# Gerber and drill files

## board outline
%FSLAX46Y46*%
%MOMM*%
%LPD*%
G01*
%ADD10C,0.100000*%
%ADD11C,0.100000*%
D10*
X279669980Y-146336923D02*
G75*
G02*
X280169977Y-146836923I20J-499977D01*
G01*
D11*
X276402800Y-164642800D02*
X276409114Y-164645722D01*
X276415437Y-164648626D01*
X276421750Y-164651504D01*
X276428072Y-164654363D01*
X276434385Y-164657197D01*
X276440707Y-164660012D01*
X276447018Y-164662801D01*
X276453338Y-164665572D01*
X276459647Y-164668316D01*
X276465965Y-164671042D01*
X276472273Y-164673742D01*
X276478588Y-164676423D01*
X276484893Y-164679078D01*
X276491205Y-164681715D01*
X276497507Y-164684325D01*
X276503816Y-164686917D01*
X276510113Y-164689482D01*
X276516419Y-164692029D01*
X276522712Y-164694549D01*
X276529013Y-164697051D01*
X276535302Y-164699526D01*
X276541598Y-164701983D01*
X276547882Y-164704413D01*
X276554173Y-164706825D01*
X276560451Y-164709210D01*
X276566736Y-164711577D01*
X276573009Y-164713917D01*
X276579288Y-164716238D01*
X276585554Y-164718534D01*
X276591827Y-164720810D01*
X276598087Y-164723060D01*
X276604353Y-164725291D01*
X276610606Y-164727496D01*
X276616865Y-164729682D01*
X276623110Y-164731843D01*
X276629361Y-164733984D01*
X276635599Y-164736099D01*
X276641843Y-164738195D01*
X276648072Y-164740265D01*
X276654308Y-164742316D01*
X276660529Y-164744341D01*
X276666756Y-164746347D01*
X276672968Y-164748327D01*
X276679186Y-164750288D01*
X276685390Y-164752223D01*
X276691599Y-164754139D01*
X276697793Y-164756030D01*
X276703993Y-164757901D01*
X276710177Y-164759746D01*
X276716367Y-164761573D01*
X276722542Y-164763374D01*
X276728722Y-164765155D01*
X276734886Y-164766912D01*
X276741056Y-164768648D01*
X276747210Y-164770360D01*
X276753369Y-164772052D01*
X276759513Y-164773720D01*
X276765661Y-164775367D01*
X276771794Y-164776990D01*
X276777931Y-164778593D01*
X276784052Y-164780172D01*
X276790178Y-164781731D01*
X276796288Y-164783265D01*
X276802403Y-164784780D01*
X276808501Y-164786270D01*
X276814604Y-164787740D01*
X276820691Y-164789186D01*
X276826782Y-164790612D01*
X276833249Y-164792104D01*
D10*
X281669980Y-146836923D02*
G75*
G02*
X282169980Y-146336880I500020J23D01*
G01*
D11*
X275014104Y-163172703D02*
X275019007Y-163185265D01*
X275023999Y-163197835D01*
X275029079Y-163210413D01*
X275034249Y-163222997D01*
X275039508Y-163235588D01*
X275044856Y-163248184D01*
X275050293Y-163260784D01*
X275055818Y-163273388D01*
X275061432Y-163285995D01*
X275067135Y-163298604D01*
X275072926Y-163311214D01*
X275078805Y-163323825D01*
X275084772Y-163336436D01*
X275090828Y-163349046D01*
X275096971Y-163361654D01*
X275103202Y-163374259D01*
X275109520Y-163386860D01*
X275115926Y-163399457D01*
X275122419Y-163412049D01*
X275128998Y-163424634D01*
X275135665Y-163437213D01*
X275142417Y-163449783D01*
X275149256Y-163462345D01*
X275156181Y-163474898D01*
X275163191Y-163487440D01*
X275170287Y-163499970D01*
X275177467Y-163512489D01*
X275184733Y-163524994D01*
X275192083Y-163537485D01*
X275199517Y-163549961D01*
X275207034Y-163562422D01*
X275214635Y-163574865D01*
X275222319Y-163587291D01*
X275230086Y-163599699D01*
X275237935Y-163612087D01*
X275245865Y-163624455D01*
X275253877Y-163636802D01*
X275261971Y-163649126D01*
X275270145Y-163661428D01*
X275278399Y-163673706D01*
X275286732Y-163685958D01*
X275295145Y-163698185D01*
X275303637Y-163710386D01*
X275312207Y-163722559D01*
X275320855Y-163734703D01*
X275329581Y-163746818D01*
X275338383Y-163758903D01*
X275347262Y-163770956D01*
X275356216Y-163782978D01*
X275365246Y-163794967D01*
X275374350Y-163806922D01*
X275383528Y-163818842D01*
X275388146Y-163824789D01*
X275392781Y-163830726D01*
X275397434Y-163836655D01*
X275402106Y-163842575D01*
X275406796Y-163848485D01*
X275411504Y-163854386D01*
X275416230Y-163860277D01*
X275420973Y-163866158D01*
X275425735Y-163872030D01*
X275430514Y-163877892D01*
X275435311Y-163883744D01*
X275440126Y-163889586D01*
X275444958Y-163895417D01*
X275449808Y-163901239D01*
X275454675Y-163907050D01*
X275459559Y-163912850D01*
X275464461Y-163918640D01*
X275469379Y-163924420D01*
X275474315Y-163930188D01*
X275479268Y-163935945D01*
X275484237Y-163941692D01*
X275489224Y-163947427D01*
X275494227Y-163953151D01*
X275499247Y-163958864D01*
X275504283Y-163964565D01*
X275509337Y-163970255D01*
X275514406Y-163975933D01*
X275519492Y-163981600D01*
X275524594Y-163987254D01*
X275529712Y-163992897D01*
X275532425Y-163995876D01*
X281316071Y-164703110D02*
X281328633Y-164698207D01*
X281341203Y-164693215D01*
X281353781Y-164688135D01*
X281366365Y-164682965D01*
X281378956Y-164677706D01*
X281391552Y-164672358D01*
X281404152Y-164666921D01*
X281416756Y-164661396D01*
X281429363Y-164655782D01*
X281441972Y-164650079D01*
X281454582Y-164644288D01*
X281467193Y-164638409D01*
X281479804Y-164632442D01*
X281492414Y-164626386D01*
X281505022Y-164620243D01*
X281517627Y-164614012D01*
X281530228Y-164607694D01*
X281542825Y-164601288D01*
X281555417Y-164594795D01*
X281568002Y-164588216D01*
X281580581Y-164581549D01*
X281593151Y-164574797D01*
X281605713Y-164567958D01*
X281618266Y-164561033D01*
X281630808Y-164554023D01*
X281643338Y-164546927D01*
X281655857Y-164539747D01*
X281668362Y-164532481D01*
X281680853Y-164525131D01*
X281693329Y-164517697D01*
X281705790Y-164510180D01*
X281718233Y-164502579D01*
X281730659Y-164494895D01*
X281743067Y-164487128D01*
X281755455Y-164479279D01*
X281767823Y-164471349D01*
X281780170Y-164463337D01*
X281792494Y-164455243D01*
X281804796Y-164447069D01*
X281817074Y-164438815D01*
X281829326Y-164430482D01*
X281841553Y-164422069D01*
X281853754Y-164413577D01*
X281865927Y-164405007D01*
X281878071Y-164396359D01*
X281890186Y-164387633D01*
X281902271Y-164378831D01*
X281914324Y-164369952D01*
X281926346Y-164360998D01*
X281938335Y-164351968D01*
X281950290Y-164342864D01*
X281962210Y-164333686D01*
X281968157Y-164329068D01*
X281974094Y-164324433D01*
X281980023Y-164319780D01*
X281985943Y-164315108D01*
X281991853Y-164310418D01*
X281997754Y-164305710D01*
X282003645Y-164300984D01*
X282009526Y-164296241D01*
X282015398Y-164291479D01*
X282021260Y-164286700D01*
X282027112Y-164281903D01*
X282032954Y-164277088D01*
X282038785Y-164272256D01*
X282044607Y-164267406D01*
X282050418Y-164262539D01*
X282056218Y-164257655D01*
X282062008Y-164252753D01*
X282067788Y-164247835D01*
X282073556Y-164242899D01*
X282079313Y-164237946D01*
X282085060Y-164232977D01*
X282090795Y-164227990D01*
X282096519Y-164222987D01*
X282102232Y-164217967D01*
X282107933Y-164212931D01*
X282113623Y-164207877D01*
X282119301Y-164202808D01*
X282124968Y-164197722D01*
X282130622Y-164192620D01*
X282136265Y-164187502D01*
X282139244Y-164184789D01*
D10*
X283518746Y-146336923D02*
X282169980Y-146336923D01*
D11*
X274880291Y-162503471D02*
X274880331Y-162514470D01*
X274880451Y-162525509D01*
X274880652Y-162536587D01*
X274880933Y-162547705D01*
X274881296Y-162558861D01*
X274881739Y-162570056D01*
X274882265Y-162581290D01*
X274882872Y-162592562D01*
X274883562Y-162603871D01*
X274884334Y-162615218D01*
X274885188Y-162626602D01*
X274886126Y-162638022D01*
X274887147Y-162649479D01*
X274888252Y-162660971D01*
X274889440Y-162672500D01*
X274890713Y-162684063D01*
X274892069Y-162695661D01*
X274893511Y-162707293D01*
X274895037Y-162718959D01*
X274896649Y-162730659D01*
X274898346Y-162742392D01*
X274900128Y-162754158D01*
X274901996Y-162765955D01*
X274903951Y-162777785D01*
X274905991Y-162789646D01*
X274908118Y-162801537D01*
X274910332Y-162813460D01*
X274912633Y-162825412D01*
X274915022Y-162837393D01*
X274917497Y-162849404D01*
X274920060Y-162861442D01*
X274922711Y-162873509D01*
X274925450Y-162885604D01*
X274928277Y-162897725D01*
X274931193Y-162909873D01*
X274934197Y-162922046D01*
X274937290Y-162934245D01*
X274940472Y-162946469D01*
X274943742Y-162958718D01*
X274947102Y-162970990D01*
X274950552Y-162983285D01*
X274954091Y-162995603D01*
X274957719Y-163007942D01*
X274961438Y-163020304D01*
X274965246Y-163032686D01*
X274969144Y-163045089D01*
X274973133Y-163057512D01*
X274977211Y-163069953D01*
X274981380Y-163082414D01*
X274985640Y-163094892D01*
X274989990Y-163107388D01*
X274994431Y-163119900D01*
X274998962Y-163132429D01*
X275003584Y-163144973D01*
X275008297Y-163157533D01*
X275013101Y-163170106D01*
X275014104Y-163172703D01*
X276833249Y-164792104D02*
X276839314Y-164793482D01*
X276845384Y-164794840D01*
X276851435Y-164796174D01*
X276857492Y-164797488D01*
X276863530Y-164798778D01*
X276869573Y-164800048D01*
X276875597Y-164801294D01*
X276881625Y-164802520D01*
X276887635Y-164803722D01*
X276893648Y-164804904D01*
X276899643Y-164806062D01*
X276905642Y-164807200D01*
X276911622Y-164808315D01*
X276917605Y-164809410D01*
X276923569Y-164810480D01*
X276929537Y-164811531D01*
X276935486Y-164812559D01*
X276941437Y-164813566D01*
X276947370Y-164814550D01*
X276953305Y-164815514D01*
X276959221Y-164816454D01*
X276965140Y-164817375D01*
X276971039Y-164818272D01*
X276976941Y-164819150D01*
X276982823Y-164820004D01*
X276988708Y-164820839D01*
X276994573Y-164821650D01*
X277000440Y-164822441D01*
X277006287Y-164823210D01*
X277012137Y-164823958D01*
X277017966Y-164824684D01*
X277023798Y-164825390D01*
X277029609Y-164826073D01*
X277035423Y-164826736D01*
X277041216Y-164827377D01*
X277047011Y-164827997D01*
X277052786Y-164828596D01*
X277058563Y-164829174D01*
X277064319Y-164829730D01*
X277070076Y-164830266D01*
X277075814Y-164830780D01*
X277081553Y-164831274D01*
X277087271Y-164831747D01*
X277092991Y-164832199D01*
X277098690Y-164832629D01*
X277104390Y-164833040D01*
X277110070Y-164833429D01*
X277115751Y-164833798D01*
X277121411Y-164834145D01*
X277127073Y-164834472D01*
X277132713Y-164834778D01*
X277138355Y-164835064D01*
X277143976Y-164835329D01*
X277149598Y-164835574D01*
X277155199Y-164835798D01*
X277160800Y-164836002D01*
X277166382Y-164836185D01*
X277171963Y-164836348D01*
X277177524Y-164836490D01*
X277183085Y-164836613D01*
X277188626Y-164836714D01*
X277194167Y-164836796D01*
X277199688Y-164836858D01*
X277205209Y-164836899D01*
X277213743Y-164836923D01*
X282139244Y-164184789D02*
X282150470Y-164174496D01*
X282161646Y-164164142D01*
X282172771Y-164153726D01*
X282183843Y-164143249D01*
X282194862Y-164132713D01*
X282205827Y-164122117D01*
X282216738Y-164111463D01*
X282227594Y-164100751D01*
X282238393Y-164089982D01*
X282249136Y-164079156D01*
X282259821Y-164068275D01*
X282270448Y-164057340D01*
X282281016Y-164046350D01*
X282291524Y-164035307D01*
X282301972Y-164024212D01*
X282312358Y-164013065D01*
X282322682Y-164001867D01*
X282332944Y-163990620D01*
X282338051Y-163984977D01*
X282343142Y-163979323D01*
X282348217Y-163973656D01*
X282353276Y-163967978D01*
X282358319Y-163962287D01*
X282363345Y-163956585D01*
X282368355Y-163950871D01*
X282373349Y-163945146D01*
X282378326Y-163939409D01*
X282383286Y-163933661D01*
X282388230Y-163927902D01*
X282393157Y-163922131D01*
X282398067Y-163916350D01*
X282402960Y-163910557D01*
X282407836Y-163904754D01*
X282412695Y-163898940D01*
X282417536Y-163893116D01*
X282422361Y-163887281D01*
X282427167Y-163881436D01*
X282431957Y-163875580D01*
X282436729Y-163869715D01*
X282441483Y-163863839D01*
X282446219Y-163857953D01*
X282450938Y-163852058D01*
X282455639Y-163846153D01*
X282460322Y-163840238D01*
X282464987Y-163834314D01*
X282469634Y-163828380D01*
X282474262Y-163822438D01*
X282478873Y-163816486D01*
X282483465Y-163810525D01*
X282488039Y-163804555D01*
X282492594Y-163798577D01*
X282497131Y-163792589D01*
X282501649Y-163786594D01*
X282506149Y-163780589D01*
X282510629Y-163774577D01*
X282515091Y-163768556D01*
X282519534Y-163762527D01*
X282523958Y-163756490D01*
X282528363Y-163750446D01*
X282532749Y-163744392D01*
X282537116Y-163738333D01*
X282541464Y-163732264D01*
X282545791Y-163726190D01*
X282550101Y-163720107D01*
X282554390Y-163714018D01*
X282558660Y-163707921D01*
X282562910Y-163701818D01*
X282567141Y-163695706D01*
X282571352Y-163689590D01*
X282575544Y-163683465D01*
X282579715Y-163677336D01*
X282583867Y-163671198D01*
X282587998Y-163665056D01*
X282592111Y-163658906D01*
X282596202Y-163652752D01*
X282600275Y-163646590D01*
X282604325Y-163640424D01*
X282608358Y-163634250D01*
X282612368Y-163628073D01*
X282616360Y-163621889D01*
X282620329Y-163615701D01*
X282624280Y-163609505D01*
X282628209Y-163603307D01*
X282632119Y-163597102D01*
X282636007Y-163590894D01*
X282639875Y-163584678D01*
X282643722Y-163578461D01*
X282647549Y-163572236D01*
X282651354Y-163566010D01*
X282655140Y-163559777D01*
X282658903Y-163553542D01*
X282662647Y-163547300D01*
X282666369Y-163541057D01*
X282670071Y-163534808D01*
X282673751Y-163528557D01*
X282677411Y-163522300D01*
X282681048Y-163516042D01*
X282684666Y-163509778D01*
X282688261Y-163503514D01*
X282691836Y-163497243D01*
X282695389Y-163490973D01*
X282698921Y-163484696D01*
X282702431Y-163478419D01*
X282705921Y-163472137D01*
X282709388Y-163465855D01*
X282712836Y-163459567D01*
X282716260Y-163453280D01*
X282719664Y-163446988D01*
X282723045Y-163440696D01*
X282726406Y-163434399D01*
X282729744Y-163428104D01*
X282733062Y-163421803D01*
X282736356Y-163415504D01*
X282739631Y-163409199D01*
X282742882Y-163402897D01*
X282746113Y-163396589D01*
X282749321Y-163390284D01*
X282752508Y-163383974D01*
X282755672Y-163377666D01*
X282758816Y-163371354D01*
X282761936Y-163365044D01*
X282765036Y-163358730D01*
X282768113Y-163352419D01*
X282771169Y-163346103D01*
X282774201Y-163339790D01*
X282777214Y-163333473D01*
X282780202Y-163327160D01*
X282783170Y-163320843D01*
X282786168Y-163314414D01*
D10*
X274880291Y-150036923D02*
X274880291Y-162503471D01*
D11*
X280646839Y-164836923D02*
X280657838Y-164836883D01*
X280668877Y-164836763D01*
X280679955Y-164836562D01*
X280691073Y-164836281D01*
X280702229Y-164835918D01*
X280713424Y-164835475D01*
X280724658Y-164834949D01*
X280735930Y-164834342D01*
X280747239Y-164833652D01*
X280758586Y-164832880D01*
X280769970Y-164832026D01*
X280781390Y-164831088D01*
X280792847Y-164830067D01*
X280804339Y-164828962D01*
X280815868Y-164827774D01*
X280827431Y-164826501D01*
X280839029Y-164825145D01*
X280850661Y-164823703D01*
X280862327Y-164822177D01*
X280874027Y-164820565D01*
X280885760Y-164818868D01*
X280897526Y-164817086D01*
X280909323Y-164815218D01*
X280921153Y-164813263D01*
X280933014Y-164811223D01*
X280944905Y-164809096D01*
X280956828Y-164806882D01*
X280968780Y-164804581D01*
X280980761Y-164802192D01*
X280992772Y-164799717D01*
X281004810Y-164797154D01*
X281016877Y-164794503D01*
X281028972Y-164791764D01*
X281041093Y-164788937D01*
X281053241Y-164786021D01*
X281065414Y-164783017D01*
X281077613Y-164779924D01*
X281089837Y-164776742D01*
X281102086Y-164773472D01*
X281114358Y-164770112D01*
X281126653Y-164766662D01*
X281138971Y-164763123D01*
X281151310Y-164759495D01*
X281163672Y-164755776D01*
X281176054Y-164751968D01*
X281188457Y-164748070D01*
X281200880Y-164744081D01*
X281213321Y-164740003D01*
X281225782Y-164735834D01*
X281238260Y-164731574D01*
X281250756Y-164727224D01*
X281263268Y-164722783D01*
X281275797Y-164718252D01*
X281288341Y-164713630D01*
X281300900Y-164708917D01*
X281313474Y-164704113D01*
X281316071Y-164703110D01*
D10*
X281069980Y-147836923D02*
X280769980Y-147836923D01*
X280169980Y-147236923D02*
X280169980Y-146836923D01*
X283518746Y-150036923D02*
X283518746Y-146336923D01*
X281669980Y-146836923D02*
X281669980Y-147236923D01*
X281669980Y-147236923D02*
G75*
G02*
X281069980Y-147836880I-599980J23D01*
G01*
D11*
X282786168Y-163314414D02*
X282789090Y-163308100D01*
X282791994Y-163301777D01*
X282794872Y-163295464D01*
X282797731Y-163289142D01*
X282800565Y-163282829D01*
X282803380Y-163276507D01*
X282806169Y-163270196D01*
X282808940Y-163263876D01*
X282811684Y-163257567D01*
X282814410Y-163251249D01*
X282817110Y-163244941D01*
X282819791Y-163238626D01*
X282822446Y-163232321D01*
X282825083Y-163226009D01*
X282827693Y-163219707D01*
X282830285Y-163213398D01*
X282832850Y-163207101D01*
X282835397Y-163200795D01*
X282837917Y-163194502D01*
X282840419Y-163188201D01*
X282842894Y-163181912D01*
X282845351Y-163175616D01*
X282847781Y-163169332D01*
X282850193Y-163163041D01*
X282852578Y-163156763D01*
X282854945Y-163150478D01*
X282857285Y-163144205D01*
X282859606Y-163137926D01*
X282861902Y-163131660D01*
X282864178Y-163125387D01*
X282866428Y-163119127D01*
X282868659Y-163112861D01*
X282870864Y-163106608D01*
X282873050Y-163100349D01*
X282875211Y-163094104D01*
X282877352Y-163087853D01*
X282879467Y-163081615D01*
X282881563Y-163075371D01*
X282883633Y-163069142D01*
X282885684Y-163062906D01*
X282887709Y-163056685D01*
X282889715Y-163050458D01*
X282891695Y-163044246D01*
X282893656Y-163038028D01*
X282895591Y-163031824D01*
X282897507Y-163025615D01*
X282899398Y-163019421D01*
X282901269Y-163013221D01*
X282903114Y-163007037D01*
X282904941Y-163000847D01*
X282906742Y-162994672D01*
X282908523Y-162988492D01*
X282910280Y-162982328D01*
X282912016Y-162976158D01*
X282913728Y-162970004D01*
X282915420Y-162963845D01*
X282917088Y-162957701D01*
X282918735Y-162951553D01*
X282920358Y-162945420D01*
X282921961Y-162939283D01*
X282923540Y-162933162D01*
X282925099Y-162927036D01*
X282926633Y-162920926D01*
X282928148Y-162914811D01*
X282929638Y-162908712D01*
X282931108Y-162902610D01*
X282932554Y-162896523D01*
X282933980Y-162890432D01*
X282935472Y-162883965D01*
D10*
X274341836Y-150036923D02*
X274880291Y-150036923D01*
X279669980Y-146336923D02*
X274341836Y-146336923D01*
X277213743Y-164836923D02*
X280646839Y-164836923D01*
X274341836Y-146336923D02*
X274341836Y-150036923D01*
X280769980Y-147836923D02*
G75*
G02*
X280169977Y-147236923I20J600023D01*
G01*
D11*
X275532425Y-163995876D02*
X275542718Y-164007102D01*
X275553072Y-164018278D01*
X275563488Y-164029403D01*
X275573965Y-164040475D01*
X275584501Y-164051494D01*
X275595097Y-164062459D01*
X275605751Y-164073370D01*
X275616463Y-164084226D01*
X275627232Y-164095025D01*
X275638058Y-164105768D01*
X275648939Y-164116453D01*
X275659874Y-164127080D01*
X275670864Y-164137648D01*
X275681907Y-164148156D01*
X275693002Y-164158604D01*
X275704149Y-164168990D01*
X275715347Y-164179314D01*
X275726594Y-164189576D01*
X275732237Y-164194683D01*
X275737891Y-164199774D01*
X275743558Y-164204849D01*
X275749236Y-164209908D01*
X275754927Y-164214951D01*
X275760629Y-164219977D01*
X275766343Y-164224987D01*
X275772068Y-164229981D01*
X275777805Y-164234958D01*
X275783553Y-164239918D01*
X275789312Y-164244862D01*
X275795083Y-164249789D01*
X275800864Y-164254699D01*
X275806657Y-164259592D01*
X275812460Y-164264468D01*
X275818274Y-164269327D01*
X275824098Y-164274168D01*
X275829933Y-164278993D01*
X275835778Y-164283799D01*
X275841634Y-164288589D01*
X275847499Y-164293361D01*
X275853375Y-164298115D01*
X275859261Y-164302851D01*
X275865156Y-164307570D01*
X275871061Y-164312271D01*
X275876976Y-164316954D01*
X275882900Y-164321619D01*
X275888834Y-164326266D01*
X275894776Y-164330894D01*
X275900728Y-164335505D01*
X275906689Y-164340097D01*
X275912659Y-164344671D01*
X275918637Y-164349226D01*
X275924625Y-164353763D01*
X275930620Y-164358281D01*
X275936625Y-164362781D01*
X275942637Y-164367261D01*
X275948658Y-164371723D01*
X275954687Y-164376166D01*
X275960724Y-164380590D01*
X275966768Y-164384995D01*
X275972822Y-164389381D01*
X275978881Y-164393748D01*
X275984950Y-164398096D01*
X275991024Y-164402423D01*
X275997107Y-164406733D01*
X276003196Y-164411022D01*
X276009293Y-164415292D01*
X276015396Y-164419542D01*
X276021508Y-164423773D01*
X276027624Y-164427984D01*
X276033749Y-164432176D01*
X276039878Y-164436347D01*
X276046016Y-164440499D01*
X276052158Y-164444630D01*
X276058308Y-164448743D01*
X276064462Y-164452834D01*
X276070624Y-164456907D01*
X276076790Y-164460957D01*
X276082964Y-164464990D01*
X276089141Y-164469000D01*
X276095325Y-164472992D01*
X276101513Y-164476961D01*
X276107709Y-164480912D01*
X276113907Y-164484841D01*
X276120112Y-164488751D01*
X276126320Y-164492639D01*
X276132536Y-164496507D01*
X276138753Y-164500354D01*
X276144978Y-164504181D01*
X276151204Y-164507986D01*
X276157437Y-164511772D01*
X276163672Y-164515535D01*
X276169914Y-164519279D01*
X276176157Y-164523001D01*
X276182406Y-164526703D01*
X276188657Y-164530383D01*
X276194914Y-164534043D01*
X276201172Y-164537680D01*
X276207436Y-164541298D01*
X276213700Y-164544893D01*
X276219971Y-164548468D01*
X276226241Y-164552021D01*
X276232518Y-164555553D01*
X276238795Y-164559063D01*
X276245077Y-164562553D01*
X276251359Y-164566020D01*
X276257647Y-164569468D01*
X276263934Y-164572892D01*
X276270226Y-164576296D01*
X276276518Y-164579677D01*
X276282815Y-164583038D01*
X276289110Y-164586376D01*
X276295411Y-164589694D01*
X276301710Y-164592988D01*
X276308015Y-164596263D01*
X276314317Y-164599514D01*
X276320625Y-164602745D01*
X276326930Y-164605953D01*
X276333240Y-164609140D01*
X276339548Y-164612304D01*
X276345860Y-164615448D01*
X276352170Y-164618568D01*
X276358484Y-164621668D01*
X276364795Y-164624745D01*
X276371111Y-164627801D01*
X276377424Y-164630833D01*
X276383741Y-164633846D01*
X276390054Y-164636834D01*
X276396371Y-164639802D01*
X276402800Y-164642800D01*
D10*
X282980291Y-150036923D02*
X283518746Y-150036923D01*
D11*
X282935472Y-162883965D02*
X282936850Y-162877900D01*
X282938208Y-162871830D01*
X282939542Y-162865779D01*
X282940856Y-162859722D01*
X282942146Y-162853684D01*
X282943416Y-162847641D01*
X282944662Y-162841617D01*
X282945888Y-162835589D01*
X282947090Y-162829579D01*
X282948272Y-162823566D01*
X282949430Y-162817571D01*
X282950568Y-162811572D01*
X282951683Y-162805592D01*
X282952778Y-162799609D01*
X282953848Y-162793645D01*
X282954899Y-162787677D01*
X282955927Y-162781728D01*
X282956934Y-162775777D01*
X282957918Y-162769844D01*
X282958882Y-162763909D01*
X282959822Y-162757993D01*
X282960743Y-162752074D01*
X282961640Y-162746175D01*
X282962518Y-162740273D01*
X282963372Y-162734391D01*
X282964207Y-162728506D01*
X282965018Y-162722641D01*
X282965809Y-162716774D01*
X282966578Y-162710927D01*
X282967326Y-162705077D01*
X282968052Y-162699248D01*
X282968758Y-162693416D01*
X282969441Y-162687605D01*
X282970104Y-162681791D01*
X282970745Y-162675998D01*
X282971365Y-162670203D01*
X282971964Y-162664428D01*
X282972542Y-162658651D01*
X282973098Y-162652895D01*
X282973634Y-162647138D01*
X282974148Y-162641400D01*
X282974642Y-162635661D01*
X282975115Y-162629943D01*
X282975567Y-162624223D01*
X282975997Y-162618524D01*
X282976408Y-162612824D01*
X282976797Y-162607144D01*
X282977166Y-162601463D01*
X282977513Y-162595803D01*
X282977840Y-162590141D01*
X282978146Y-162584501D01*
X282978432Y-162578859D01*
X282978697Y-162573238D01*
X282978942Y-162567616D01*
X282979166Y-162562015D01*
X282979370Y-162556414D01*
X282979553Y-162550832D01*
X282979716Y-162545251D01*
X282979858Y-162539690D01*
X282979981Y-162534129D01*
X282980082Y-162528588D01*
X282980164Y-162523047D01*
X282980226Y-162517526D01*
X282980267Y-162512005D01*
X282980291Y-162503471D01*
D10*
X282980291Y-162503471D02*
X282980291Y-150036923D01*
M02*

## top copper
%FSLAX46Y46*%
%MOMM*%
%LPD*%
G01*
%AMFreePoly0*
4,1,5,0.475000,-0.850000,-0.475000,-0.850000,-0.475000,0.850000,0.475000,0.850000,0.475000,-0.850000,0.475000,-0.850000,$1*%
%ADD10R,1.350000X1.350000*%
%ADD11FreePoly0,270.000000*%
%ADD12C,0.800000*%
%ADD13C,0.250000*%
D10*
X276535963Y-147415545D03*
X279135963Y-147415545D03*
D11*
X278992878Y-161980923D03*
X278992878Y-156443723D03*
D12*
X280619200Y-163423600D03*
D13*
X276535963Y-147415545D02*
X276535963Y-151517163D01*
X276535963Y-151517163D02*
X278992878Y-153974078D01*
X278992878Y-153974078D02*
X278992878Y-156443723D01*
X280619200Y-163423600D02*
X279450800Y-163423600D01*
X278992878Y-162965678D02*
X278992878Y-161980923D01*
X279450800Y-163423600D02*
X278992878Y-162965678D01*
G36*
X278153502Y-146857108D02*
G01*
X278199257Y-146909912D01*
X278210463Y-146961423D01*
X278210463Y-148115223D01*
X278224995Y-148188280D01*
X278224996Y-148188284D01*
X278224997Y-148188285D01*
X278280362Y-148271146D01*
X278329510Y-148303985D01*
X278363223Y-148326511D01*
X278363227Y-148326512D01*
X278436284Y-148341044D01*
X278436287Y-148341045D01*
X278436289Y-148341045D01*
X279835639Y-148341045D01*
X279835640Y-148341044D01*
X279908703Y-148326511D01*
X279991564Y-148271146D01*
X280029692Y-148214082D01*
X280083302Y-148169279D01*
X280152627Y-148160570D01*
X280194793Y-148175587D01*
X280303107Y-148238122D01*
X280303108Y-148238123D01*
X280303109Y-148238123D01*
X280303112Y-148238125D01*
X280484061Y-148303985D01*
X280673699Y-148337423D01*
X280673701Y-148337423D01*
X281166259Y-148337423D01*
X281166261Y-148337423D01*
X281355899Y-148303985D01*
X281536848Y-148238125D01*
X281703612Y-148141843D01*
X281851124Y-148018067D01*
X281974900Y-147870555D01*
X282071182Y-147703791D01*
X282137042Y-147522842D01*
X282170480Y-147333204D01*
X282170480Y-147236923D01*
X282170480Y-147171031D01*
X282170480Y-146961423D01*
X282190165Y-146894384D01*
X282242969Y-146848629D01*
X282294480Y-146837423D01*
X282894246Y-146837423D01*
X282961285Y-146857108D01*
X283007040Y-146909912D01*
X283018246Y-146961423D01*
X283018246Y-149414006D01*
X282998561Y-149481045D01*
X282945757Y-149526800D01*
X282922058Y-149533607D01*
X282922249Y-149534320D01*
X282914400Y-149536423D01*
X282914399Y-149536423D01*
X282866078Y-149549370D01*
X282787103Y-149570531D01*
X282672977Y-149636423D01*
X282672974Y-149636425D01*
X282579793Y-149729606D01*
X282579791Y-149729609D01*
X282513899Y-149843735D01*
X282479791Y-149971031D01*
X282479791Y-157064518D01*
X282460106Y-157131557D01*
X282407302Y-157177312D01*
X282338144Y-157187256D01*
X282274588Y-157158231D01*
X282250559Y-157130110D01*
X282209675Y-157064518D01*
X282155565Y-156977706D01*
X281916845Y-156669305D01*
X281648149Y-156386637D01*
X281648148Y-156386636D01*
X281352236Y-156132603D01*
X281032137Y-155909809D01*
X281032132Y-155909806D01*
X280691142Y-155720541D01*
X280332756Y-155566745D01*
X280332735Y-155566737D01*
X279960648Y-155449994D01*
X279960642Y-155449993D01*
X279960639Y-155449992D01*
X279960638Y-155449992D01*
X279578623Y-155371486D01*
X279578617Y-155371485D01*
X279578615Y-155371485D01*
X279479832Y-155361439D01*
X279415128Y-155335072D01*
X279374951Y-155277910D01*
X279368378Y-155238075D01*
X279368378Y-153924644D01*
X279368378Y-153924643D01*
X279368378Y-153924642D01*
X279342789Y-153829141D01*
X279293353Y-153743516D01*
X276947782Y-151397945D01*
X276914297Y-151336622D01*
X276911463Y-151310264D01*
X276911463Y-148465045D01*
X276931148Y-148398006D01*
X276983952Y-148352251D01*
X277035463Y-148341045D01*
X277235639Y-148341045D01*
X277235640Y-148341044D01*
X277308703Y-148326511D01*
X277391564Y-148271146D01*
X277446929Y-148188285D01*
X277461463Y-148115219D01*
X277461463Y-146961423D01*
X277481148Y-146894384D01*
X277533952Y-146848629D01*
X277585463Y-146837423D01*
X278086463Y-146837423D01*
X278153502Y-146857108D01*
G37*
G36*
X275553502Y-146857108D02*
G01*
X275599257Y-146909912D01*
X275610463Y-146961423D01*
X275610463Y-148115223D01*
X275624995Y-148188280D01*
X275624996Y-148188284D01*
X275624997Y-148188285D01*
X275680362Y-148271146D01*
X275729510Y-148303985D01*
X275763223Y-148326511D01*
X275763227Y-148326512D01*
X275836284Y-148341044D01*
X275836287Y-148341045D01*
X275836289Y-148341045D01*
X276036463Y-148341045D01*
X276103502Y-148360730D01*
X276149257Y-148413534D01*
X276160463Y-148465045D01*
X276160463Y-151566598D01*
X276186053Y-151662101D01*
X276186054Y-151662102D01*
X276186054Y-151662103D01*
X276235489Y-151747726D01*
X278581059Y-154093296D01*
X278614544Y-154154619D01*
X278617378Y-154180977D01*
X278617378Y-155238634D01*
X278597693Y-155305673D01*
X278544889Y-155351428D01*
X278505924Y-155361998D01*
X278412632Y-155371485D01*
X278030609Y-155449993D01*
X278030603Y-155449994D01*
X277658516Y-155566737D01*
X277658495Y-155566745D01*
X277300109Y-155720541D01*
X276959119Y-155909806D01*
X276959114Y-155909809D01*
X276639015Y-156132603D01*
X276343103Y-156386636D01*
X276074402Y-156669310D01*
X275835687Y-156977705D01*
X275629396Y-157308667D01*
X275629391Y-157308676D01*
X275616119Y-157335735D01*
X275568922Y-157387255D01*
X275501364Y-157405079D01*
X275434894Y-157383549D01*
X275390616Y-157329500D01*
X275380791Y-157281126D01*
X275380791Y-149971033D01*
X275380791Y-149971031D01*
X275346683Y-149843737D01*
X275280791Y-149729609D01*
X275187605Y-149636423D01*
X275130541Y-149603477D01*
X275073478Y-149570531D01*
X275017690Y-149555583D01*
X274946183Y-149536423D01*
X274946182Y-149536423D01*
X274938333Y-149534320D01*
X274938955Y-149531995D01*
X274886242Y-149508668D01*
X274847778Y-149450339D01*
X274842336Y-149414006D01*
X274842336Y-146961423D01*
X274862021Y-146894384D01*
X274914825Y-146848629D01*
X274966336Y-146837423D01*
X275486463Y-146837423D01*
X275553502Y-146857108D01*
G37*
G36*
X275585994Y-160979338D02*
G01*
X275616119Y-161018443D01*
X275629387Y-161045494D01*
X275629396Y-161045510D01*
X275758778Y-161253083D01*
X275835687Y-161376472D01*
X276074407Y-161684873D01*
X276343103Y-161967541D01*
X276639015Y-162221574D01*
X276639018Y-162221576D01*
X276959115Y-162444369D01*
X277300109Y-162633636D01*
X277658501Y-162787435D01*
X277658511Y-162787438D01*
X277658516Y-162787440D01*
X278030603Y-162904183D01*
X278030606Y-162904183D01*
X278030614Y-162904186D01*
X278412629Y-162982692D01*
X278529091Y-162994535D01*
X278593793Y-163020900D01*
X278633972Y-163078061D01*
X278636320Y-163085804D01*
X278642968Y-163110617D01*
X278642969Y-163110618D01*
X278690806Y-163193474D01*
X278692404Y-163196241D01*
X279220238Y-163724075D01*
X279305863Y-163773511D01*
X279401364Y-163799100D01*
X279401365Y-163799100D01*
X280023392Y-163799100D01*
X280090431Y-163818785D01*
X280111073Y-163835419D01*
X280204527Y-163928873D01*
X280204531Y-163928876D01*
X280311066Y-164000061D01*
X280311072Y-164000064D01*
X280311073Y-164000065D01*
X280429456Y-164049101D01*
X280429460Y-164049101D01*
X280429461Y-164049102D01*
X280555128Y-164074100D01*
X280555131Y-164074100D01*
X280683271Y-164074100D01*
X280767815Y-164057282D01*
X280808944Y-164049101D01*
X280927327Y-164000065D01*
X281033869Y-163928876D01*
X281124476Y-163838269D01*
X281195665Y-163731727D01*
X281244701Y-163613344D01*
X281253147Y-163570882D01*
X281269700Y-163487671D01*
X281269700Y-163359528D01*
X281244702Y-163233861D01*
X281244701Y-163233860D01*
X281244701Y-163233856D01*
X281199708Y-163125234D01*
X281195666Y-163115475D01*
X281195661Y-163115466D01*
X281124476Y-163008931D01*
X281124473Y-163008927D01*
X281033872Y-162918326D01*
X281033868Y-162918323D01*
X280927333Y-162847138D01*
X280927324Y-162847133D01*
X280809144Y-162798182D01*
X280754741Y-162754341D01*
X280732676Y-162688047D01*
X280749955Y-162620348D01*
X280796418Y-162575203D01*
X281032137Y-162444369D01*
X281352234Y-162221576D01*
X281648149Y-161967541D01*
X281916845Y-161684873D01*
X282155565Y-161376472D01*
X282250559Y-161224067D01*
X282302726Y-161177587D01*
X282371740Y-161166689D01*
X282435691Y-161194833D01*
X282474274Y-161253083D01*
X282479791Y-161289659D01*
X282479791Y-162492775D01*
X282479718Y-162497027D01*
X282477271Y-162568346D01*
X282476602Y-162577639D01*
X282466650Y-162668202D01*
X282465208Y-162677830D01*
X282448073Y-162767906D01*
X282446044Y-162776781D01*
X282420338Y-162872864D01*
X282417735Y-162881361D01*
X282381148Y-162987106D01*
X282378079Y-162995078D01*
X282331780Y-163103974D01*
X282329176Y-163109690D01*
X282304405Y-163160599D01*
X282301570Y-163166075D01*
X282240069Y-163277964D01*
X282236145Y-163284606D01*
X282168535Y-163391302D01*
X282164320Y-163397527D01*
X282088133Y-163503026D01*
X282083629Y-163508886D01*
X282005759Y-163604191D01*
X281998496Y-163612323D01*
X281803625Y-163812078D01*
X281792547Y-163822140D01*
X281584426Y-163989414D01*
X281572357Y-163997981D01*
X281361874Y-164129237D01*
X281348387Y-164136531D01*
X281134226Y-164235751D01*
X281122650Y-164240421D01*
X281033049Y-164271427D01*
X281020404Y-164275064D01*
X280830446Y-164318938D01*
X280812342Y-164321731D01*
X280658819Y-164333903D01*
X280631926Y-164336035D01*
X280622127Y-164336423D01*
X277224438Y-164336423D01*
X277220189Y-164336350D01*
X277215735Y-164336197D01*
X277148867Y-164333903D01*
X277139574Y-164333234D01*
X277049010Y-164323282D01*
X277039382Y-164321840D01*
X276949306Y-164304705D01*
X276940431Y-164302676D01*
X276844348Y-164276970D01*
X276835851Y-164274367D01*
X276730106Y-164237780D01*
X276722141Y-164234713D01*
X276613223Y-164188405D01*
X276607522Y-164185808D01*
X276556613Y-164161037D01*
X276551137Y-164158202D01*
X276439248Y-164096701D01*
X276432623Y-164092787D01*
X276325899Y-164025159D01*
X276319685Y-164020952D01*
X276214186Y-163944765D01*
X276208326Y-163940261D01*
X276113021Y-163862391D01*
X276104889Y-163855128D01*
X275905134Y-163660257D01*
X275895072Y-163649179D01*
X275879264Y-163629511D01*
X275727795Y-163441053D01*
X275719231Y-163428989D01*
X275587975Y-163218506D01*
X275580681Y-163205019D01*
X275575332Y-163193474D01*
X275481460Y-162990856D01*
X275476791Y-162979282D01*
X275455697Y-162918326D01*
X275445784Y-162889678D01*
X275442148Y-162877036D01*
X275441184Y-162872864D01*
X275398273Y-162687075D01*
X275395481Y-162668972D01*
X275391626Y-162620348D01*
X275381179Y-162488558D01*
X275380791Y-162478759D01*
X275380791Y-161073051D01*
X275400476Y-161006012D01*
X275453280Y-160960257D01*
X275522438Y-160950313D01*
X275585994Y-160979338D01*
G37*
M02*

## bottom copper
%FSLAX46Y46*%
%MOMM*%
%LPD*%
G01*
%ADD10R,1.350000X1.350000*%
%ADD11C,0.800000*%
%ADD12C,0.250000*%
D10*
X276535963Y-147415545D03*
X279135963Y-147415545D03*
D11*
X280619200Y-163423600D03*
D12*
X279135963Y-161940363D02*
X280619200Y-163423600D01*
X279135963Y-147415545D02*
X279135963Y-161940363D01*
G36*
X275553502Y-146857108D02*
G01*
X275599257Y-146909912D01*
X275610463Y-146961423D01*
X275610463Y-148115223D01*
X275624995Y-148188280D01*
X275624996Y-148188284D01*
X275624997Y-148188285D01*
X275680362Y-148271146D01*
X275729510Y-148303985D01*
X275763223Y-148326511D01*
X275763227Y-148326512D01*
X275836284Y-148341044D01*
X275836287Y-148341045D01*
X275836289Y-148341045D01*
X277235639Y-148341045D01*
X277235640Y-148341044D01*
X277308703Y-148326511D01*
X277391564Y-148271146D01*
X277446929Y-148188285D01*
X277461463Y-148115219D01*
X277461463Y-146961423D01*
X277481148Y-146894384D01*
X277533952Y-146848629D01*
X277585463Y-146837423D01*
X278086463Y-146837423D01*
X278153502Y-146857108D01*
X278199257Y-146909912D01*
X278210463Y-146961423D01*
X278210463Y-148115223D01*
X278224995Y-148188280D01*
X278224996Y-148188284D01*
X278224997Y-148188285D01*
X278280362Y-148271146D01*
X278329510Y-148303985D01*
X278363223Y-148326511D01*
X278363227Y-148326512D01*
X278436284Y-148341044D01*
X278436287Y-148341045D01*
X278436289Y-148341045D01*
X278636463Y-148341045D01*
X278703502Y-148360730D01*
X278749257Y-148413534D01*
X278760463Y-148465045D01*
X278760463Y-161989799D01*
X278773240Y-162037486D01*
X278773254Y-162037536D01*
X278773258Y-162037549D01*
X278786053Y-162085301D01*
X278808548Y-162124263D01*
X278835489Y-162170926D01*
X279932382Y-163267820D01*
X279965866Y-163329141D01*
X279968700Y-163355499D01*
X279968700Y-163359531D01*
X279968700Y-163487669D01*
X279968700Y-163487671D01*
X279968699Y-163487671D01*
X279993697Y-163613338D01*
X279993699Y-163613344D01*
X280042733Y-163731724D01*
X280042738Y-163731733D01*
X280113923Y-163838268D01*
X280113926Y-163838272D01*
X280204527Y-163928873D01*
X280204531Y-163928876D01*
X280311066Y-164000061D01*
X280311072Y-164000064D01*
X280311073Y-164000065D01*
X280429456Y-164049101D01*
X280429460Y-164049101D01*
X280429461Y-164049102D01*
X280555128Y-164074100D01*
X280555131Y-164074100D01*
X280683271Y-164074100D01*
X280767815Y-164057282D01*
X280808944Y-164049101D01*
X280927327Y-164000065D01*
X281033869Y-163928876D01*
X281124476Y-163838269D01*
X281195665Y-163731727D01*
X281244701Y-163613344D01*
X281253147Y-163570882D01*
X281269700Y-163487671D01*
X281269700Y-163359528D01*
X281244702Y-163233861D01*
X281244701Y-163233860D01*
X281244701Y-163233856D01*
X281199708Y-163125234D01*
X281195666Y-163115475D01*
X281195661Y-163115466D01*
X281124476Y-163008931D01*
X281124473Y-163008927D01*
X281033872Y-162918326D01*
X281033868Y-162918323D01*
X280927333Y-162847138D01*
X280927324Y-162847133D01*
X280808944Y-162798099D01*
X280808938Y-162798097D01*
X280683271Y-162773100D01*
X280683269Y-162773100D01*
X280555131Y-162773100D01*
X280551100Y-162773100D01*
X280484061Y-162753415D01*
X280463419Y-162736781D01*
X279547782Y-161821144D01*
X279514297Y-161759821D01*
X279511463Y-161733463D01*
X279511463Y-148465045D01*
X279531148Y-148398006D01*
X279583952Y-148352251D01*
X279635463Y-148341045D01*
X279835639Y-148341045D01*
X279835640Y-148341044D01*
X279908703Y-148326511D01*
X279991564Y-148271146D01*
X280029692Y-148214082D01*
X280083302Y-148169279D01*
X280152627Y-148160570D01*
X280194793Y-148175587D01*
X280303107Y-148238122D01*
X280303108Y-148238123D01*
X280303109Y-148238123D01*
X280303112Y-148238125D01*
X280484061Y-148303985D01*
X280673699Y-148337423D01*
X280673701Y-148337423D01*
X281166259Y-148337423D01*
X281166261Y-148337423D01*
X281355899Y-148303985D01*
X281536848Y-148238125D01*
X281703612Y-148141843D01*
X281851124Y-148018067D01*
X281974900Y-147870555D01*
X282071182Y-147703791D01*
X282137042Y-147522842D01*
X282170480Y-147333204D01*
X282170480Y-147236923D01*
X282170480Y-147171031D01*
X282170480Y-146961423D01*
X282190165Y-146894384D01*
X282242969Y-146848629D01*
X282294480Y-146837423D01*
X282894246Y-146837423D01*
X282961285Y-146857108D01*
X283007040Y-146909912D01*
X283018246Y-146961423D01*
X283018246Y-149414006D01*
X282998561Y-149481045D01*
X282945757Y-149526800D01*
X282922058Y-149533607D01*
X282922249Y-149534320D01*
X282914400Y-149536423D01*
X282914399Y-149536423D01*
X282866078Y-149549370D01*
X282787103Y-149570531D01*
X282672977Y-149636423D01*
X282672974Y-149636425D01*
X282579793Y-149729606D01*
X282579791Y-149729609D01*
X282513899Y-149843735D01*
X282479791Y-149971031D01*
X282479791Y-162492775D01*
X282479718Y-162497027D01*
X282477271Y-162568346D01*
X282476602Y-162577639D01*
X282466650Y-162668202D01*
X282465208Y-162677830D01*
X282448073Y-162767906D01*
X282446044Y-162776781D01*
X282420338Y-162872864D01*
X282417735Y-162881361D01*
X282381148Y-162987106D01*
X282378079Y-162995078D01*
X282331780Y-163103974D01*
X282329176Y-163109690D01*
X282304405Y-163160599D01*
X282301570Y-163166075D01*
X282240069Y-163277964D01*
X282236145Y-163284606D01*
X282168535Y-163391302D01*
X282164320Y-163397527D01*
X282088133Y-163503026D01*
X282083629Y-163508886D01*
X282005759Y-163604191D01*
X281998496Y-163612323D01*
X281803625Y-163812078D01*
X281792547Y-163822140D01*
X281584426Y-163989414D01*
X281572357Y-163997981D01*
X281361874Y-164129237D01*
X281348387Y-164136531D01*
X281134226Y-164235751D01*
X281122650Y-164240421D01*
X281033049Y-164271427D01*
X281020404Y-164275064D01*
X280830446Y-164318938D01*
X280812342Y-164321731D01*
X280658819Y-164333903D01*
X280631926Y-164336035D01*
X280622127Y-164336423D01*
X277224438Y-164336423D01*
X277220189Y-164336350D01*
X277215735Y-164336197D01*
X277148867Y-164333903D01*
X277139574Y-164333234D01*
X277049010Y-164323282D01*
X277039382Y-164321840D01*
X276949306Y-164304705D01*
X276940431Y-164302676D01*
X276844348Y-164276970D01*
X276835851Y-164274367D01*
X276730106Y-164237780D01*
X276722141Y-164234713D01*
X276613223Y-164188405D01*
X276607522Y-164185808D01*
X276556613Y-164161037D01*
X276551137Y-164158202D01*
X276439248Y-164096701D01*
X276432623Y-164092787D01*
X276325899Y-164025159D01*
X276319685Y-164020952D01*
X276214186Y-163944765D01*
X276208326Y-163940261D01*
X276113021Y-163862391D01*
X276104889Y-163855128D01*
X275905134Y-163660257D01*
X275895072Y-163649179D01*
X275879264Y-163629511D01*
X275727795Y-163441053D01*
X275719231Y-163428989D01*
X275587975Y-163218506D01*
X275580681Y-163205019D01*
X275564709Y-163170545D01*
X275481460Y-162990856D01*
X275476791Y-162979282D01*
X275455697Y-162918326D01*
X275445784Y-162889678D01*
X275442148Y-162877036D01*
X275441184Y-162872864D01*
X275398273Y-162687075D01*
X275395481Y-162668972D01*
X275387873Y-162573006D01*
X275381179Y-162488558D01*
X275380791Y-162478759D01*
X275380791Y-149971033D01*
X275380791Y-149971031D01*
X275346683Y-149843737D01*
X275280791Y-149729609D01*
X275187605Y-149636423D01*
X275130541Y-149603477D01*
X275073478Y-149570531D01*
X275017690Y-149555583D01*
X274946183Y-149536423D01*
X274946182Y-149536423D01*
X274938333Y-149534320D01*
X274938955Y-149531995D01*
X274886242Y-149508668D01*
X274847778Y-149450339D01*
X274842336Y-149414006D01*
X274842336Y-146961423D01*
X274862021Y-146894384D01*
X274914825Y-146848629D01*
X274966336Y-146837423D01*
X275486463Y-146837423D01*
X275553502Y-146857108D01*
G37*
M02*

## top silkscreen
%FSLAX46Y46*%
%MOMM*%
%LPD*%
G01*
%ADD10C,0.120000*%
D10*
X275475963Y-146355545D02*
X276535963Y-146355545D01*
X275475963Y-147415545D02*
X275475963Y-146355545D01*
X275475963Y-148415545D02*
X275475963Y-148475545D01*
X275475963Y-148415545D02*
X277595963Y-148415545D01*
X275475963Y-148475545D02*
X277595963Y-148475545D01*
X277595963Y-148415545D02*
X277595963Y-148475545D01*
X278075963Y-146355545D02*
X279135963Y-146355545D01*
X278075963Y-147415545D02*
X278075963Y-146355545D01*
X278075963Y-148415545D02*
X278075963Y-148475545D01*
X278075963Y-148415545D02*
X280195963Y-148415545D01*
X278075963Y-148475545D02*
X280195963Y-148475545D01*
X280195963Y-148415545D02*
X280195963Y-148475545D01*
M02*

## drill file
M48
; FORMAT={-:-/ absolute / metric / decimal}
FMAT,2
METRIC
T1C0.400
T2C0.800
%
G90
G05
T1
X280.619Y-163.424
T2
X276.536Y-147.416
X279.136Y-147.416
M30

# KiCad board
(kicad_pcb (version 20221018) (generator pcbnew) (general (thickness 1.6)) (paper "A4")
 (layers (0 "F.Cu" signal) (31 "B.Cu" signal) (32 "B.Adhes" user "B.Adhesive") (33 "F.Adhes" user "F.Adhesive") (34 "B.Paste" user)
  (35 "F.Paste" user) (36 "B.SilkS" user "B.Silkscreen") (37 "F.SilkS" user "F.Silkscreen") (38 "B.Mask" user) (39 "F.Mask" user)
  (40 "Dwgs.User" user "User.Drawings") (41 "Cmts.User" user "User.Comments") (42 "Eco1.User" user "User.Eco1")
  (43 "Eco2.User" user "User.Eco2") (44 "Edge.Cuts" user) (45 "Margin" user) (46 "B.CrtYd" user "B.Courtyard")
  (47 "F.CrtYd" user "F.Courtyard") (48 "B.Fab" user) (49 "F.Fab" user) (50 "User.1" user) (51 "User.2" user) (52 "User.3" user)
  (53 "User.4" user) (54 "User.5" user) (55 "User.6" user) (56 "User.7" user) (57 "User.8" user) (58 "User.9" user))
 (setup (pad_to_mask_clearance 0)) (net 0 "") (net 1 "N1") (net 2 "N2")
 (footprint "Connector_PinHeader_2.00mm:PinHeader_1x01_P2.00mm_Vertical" (layer "F.Cu") (at 276.535963 147.415545)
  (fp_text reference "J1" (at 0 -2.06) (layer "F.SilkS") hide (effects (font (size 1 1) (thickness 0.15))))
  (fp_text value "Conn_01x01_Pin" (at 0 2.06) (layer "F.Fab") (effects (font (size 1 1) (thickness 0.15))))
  (fp_line (start -1.06 -1.06) (end 0 -1.06) (stroke (width 0.12) (type solid)) (layer "F.SilkS"))
  (fp_line (start -1.06 0) (end -1.06 -1.06) (stroke (width 0.12) (type solid)) (layer "F.SilkS"))
  (fp_line (start -1.06 1) (end -1.06 1.06) (stroke (width 0.12) (type solid)) (layer "F.SilkS"))
  (fp_line (start -1.06 1) (end 1.06 1) (stroke (width 0.12) (type solid)) (layer "F.SilkS"))
  (fp_line (start -1.06 1.06) (end 1.06 1.06) (stroke (width 0.12) (type solid)) (layer "F.SilkS"))
  (fp_line (start 1.06 1) (end 1.06 1.06) (stroke (width 0.12) (type solid)) (layer "F.SilkS"))
  (pad "1" thru_hole rect (at 0 0) (size 1.35 1.35) (drill 0.8) (layers "*.Cu" "*.Mask") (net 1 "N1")))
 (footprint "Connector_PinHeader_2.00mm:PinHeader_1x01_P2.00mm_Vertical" (layer "F.Cu") (at 279.135963 147.415545)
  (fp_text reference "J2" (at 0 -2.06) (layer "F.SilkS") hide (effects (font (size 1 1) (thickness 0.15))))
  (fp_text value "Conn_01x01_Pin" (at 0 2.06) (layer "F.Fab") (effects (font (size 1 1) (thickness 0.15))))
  (fp_line (start -1.06 -1.06) (end 0 -1.06) (stroke (width 0.12) (type solid)) (layer "F.SilkS"))
  (fp_line (start -1.06 0) (end -1.06 -1.06) (stroke (width 0.12) (type solid)) (layer "F.SilkS"))
  (fp_line (start -1.06 1) (end -1.06 1.06) (stroke (width 0.12) (type solid)) (layer "F.SilkS"))
  (fp_line (start -1.06 1) (end 1.06 1) (stroke (width 0.12) (type solid)) (layer "F.SilkS"))
  (fp_line (start -1.06 1.06) (end 1.06 1.06) (stroke (width 0.12) (type solid)) (layer "F.SilkS"))
  (fp_line (start 1.06 1) (end 1.06 1.06) (stroke (width 0.12) (type solid)) (layer "F.SilkS"))
  (pad "1" thru_hole rect (at 0 0) (size 1.35 1.35) (drill 0.8) (layers "*.Cu" "*.Mask") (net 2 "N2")))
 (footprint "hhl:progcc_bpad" (layer "F.Cu") (at 278.992878 159.186923)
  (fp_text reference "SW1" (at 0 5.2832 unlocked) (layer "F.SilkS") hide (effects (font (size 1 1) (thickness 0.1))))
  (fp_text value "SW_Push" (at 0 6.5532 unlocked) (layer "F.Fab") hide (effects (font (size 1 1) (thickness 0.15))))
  (pad "1" smd custom (at 0 2.794 270) (size 0.95 1.7) (layers "F.Cu") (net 2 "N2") (thermal_bridge_angle 45)
   (options (clearance outline) (anchor rect)) (primitives))
  (pad "2" smd custom (at 0 -2.7432 270) (size 0.95 1.7) (layers "F.Cu") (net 1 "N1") (thermal_bridge_angle 45)
   (options (clearance outline) (anchor rect)) (primitives))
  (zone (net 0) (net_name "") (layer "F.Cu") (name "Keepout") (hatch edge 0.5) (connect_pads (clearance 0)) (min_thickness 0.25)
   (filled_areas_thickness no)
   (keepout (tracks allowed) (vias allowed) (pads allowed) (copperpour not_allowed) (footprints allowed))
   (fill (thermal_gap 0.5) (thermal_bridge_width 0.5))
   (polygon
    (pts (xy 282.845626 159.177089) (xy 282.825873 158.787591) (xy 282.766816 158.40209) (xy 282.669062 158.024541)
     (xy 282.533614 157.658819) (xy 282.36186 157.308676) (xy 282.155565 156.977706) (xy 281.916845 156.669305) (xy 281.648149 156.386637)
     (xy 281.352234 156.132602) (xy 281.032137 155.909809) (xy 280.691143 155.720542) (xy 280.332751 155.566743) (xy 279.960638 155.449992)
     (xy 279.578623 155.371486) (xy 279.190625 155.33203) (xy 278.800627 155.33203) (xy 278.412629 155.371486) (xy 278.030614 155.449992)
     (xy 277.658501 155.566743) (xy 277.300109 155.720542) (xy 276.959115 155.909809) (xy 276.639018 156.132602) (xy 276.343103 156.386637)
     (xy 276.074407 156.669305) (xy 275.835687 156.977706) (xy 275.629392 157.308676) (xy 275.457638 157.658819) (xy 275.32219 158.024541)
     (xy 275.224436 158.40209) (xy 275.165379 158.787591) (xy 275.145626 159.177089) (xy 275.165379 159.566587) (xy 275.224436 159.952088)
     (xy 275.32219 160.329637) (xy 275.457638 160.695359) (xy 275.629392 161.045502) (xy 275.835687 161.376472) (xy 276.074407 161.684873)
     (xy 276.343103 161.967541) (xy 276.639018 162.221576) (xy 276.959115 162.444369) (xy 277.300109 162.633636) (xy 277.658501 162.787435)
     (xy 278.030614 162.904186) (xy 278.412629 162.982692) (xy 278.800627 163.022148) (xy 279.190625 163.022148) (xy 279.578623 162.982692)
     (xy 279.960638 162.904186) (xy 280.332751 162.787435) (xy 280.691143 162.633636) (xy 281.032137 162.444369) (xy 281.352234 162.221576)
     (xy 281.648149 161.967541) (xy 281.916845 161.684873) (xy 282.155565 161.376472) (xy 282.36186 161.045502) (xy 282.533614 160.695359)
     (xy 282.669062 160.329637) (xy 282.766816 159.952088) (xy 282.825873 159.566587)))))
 (gr_arc (start 279.66998 146.336923) (mid 280.023533 146.48337) (end 280.16998 146.836923) (stroke (width 0.1) (type solid))
  (layer "Edge.Cuts"))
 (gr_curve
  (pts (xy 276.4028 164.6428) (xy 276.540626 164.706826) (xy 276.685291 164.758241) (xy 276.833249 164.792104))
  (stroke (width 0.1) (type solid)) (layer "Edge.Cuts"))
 (gr_arc (start 281.66998 146.836923) (mid 281.816427 146.48337) (end 282.16998 146.336923) (stroke (width 0.1) (type solid))
  (layer "Edge.Cuts"))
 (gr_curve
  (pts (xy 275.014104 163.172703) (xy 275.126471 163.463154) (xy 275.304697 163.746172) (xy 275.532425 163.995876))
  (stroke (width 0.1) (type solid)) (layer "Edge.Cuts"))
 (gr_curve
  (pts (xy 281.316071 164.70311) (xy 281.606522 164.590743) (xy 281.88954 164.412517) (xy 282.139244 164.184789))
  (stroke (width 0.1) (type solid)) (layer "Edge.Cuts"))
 (gr_line (start 283.518746 146.336923) (end 282.16998 146.336923) (stroke (width 0.1) (type solid)) (layer "Edge.Cuts"))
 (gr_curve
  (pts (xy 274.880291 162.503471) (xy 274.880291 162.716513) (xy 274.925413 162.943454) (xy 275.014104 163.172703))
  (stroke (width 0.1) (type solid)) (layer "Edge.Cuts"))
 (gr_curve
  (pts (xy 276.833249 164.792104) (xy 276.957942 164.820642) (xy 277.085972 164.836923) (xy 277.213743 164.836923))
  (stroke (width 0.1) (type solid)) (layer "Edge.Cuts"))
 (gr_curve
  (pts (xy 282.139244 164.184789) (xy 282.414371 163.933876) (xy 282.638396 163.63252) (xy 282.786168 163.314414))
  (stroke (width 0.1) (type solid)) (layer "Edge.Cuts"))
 (gr_line (start 274.880291 150.036923) (end 274.880291 162.503471) (stroke (width 0.1) (type solid)) (layer "Edge.Cuts"))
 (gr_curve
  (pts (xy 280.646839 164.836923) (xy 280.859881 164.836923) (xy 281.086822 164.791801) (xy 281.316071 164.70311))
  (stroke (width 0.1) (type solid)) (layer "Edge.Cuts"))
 (gr_line (start 281.06998 147.836923) (end 280.76998 147.836923) (stroke (width 0.1) (type solid)) (layer "Edge.Cuts"))
 (gr_line (start 280.16998 147.236923) (end 280.16998 146.836923) (stroke (width 0.1) (type solid)) (layer "Edge.Cuts"))
 (gr_line (start 283.518746 150.036923) (end 283.518746 146.336923) (stroke (width 0.1) (type solid)) (layer "Edge.Cuts"))
 (gr_line (start 281.66998 146.836923) (end 281.66998 147.236923) (stroke (width 0.1) (type solid)) (layer "Edge.Cuts"))
 (gr_arc (start 281.66998 147.236923) (mid 281.494244 147.661187) (end 281.06998 147.836923) (stroke (width 0.1) (type solid))
  (layer "Edge.Cuts"))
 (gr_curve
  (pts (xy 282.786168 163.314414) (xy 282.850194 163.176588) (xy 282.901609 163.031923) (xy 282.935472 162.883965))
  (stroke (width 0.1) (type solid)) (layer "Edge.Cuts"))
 (gr_line (start 274.341836 150.036923) (end 274.880291 150.036923) (stroke (width 0.1) (type solid)) (layer "Edge.Cuts"))
 (gr_line (start 279.66998 146.336923) (end 274.341836 146.336923) (stroke (width 0.1) (type solid)) (layer "Edge.Cuts"))
 (gr_line (start 277.213743 164.836923) (end 280.646839 164.836923) (stroke (width 0.1) (type solid)) (layer "Edge.Cuts"))
 (gr_line (start 274.341836 146.336923) (end 274.341836 150.036923) (stroke (width 0.1) (type solid)) (layer "Edge.Cuts"))
 (gr_arc (start 280.76998 147.836923) (mid 280.345716 147.661187) (end 280.16998 147.236923) (stroke (width 0.1) (type solid))
  (layer "Edge.Cuts"))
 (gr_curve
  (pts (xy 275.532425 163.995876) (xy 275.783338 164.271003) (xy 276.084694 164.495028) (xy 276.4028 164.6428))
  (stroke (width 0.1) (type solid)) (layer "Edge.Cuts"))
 (gr_line (start 282.980291 150.036923) (end 283.518746 150.036923) (stroke (width 0.1) (type solid)) (layer "Edge.Cuts"))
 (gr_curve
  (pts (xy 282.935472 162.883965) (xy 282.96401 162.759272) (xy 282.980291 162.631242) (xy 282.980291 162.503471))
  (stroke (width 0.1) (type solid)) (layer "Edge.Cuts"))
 (gr_line (start 282.980291 162.503471) (end 282.980291 150.036923) (stroke (width 0.1) (type solid)) (layer "Edge.Cuts"))
 (segment (start 276.535963 147.415545) (end 276.535963 151.517163) (width 0.25) (layer "F.Cu") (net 1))
 (segment (start 276.535963 151.517163) (end 278.992878 153.974078) (width 0.25) (layer "F.Cu") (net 1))
 (segment (start 278.992878 153.974078) (end 278.992878 156.443723) (width 0.25) (layer "F.Cu") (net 1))
 (segment (start 280.6192 163.4236) (end 279.4508 163.4236) (width 0.25) (layer "F.Cu") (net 2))
 (segment (start 278.992878 162.965678) (end 278.992878 161.980923) (width 0.25) (layer "F.Cu") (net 2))
 (segment (start 279.4508 163.4236) (end 278.992878 162.965678) (width 0.25) (layer "F.Cu") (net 2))
 (via (at 280.6192 163.4236) (size 0.8) (drill 0.4) (layers "F.Cu" "B.Cu") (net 2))
 (segment (start 279.135963 161.940363) (end 280.6192 163.4236) (width 0.25) (layer "B.Cu") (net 2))
 (segment (start 279.135963 147.415545) (end 279.135963 161.940363) (width 0.25) (layer "B.Cu") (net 2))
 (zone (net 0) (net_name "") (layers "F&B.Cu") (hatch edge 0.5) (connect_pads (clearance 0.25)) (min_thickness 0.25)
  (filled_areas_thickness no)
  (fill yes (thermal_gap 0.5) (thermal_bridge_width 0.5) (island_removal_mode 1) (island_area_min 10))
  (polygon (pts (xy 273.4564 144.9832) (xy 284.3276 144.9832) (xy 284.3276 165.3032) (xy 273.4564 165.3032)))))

